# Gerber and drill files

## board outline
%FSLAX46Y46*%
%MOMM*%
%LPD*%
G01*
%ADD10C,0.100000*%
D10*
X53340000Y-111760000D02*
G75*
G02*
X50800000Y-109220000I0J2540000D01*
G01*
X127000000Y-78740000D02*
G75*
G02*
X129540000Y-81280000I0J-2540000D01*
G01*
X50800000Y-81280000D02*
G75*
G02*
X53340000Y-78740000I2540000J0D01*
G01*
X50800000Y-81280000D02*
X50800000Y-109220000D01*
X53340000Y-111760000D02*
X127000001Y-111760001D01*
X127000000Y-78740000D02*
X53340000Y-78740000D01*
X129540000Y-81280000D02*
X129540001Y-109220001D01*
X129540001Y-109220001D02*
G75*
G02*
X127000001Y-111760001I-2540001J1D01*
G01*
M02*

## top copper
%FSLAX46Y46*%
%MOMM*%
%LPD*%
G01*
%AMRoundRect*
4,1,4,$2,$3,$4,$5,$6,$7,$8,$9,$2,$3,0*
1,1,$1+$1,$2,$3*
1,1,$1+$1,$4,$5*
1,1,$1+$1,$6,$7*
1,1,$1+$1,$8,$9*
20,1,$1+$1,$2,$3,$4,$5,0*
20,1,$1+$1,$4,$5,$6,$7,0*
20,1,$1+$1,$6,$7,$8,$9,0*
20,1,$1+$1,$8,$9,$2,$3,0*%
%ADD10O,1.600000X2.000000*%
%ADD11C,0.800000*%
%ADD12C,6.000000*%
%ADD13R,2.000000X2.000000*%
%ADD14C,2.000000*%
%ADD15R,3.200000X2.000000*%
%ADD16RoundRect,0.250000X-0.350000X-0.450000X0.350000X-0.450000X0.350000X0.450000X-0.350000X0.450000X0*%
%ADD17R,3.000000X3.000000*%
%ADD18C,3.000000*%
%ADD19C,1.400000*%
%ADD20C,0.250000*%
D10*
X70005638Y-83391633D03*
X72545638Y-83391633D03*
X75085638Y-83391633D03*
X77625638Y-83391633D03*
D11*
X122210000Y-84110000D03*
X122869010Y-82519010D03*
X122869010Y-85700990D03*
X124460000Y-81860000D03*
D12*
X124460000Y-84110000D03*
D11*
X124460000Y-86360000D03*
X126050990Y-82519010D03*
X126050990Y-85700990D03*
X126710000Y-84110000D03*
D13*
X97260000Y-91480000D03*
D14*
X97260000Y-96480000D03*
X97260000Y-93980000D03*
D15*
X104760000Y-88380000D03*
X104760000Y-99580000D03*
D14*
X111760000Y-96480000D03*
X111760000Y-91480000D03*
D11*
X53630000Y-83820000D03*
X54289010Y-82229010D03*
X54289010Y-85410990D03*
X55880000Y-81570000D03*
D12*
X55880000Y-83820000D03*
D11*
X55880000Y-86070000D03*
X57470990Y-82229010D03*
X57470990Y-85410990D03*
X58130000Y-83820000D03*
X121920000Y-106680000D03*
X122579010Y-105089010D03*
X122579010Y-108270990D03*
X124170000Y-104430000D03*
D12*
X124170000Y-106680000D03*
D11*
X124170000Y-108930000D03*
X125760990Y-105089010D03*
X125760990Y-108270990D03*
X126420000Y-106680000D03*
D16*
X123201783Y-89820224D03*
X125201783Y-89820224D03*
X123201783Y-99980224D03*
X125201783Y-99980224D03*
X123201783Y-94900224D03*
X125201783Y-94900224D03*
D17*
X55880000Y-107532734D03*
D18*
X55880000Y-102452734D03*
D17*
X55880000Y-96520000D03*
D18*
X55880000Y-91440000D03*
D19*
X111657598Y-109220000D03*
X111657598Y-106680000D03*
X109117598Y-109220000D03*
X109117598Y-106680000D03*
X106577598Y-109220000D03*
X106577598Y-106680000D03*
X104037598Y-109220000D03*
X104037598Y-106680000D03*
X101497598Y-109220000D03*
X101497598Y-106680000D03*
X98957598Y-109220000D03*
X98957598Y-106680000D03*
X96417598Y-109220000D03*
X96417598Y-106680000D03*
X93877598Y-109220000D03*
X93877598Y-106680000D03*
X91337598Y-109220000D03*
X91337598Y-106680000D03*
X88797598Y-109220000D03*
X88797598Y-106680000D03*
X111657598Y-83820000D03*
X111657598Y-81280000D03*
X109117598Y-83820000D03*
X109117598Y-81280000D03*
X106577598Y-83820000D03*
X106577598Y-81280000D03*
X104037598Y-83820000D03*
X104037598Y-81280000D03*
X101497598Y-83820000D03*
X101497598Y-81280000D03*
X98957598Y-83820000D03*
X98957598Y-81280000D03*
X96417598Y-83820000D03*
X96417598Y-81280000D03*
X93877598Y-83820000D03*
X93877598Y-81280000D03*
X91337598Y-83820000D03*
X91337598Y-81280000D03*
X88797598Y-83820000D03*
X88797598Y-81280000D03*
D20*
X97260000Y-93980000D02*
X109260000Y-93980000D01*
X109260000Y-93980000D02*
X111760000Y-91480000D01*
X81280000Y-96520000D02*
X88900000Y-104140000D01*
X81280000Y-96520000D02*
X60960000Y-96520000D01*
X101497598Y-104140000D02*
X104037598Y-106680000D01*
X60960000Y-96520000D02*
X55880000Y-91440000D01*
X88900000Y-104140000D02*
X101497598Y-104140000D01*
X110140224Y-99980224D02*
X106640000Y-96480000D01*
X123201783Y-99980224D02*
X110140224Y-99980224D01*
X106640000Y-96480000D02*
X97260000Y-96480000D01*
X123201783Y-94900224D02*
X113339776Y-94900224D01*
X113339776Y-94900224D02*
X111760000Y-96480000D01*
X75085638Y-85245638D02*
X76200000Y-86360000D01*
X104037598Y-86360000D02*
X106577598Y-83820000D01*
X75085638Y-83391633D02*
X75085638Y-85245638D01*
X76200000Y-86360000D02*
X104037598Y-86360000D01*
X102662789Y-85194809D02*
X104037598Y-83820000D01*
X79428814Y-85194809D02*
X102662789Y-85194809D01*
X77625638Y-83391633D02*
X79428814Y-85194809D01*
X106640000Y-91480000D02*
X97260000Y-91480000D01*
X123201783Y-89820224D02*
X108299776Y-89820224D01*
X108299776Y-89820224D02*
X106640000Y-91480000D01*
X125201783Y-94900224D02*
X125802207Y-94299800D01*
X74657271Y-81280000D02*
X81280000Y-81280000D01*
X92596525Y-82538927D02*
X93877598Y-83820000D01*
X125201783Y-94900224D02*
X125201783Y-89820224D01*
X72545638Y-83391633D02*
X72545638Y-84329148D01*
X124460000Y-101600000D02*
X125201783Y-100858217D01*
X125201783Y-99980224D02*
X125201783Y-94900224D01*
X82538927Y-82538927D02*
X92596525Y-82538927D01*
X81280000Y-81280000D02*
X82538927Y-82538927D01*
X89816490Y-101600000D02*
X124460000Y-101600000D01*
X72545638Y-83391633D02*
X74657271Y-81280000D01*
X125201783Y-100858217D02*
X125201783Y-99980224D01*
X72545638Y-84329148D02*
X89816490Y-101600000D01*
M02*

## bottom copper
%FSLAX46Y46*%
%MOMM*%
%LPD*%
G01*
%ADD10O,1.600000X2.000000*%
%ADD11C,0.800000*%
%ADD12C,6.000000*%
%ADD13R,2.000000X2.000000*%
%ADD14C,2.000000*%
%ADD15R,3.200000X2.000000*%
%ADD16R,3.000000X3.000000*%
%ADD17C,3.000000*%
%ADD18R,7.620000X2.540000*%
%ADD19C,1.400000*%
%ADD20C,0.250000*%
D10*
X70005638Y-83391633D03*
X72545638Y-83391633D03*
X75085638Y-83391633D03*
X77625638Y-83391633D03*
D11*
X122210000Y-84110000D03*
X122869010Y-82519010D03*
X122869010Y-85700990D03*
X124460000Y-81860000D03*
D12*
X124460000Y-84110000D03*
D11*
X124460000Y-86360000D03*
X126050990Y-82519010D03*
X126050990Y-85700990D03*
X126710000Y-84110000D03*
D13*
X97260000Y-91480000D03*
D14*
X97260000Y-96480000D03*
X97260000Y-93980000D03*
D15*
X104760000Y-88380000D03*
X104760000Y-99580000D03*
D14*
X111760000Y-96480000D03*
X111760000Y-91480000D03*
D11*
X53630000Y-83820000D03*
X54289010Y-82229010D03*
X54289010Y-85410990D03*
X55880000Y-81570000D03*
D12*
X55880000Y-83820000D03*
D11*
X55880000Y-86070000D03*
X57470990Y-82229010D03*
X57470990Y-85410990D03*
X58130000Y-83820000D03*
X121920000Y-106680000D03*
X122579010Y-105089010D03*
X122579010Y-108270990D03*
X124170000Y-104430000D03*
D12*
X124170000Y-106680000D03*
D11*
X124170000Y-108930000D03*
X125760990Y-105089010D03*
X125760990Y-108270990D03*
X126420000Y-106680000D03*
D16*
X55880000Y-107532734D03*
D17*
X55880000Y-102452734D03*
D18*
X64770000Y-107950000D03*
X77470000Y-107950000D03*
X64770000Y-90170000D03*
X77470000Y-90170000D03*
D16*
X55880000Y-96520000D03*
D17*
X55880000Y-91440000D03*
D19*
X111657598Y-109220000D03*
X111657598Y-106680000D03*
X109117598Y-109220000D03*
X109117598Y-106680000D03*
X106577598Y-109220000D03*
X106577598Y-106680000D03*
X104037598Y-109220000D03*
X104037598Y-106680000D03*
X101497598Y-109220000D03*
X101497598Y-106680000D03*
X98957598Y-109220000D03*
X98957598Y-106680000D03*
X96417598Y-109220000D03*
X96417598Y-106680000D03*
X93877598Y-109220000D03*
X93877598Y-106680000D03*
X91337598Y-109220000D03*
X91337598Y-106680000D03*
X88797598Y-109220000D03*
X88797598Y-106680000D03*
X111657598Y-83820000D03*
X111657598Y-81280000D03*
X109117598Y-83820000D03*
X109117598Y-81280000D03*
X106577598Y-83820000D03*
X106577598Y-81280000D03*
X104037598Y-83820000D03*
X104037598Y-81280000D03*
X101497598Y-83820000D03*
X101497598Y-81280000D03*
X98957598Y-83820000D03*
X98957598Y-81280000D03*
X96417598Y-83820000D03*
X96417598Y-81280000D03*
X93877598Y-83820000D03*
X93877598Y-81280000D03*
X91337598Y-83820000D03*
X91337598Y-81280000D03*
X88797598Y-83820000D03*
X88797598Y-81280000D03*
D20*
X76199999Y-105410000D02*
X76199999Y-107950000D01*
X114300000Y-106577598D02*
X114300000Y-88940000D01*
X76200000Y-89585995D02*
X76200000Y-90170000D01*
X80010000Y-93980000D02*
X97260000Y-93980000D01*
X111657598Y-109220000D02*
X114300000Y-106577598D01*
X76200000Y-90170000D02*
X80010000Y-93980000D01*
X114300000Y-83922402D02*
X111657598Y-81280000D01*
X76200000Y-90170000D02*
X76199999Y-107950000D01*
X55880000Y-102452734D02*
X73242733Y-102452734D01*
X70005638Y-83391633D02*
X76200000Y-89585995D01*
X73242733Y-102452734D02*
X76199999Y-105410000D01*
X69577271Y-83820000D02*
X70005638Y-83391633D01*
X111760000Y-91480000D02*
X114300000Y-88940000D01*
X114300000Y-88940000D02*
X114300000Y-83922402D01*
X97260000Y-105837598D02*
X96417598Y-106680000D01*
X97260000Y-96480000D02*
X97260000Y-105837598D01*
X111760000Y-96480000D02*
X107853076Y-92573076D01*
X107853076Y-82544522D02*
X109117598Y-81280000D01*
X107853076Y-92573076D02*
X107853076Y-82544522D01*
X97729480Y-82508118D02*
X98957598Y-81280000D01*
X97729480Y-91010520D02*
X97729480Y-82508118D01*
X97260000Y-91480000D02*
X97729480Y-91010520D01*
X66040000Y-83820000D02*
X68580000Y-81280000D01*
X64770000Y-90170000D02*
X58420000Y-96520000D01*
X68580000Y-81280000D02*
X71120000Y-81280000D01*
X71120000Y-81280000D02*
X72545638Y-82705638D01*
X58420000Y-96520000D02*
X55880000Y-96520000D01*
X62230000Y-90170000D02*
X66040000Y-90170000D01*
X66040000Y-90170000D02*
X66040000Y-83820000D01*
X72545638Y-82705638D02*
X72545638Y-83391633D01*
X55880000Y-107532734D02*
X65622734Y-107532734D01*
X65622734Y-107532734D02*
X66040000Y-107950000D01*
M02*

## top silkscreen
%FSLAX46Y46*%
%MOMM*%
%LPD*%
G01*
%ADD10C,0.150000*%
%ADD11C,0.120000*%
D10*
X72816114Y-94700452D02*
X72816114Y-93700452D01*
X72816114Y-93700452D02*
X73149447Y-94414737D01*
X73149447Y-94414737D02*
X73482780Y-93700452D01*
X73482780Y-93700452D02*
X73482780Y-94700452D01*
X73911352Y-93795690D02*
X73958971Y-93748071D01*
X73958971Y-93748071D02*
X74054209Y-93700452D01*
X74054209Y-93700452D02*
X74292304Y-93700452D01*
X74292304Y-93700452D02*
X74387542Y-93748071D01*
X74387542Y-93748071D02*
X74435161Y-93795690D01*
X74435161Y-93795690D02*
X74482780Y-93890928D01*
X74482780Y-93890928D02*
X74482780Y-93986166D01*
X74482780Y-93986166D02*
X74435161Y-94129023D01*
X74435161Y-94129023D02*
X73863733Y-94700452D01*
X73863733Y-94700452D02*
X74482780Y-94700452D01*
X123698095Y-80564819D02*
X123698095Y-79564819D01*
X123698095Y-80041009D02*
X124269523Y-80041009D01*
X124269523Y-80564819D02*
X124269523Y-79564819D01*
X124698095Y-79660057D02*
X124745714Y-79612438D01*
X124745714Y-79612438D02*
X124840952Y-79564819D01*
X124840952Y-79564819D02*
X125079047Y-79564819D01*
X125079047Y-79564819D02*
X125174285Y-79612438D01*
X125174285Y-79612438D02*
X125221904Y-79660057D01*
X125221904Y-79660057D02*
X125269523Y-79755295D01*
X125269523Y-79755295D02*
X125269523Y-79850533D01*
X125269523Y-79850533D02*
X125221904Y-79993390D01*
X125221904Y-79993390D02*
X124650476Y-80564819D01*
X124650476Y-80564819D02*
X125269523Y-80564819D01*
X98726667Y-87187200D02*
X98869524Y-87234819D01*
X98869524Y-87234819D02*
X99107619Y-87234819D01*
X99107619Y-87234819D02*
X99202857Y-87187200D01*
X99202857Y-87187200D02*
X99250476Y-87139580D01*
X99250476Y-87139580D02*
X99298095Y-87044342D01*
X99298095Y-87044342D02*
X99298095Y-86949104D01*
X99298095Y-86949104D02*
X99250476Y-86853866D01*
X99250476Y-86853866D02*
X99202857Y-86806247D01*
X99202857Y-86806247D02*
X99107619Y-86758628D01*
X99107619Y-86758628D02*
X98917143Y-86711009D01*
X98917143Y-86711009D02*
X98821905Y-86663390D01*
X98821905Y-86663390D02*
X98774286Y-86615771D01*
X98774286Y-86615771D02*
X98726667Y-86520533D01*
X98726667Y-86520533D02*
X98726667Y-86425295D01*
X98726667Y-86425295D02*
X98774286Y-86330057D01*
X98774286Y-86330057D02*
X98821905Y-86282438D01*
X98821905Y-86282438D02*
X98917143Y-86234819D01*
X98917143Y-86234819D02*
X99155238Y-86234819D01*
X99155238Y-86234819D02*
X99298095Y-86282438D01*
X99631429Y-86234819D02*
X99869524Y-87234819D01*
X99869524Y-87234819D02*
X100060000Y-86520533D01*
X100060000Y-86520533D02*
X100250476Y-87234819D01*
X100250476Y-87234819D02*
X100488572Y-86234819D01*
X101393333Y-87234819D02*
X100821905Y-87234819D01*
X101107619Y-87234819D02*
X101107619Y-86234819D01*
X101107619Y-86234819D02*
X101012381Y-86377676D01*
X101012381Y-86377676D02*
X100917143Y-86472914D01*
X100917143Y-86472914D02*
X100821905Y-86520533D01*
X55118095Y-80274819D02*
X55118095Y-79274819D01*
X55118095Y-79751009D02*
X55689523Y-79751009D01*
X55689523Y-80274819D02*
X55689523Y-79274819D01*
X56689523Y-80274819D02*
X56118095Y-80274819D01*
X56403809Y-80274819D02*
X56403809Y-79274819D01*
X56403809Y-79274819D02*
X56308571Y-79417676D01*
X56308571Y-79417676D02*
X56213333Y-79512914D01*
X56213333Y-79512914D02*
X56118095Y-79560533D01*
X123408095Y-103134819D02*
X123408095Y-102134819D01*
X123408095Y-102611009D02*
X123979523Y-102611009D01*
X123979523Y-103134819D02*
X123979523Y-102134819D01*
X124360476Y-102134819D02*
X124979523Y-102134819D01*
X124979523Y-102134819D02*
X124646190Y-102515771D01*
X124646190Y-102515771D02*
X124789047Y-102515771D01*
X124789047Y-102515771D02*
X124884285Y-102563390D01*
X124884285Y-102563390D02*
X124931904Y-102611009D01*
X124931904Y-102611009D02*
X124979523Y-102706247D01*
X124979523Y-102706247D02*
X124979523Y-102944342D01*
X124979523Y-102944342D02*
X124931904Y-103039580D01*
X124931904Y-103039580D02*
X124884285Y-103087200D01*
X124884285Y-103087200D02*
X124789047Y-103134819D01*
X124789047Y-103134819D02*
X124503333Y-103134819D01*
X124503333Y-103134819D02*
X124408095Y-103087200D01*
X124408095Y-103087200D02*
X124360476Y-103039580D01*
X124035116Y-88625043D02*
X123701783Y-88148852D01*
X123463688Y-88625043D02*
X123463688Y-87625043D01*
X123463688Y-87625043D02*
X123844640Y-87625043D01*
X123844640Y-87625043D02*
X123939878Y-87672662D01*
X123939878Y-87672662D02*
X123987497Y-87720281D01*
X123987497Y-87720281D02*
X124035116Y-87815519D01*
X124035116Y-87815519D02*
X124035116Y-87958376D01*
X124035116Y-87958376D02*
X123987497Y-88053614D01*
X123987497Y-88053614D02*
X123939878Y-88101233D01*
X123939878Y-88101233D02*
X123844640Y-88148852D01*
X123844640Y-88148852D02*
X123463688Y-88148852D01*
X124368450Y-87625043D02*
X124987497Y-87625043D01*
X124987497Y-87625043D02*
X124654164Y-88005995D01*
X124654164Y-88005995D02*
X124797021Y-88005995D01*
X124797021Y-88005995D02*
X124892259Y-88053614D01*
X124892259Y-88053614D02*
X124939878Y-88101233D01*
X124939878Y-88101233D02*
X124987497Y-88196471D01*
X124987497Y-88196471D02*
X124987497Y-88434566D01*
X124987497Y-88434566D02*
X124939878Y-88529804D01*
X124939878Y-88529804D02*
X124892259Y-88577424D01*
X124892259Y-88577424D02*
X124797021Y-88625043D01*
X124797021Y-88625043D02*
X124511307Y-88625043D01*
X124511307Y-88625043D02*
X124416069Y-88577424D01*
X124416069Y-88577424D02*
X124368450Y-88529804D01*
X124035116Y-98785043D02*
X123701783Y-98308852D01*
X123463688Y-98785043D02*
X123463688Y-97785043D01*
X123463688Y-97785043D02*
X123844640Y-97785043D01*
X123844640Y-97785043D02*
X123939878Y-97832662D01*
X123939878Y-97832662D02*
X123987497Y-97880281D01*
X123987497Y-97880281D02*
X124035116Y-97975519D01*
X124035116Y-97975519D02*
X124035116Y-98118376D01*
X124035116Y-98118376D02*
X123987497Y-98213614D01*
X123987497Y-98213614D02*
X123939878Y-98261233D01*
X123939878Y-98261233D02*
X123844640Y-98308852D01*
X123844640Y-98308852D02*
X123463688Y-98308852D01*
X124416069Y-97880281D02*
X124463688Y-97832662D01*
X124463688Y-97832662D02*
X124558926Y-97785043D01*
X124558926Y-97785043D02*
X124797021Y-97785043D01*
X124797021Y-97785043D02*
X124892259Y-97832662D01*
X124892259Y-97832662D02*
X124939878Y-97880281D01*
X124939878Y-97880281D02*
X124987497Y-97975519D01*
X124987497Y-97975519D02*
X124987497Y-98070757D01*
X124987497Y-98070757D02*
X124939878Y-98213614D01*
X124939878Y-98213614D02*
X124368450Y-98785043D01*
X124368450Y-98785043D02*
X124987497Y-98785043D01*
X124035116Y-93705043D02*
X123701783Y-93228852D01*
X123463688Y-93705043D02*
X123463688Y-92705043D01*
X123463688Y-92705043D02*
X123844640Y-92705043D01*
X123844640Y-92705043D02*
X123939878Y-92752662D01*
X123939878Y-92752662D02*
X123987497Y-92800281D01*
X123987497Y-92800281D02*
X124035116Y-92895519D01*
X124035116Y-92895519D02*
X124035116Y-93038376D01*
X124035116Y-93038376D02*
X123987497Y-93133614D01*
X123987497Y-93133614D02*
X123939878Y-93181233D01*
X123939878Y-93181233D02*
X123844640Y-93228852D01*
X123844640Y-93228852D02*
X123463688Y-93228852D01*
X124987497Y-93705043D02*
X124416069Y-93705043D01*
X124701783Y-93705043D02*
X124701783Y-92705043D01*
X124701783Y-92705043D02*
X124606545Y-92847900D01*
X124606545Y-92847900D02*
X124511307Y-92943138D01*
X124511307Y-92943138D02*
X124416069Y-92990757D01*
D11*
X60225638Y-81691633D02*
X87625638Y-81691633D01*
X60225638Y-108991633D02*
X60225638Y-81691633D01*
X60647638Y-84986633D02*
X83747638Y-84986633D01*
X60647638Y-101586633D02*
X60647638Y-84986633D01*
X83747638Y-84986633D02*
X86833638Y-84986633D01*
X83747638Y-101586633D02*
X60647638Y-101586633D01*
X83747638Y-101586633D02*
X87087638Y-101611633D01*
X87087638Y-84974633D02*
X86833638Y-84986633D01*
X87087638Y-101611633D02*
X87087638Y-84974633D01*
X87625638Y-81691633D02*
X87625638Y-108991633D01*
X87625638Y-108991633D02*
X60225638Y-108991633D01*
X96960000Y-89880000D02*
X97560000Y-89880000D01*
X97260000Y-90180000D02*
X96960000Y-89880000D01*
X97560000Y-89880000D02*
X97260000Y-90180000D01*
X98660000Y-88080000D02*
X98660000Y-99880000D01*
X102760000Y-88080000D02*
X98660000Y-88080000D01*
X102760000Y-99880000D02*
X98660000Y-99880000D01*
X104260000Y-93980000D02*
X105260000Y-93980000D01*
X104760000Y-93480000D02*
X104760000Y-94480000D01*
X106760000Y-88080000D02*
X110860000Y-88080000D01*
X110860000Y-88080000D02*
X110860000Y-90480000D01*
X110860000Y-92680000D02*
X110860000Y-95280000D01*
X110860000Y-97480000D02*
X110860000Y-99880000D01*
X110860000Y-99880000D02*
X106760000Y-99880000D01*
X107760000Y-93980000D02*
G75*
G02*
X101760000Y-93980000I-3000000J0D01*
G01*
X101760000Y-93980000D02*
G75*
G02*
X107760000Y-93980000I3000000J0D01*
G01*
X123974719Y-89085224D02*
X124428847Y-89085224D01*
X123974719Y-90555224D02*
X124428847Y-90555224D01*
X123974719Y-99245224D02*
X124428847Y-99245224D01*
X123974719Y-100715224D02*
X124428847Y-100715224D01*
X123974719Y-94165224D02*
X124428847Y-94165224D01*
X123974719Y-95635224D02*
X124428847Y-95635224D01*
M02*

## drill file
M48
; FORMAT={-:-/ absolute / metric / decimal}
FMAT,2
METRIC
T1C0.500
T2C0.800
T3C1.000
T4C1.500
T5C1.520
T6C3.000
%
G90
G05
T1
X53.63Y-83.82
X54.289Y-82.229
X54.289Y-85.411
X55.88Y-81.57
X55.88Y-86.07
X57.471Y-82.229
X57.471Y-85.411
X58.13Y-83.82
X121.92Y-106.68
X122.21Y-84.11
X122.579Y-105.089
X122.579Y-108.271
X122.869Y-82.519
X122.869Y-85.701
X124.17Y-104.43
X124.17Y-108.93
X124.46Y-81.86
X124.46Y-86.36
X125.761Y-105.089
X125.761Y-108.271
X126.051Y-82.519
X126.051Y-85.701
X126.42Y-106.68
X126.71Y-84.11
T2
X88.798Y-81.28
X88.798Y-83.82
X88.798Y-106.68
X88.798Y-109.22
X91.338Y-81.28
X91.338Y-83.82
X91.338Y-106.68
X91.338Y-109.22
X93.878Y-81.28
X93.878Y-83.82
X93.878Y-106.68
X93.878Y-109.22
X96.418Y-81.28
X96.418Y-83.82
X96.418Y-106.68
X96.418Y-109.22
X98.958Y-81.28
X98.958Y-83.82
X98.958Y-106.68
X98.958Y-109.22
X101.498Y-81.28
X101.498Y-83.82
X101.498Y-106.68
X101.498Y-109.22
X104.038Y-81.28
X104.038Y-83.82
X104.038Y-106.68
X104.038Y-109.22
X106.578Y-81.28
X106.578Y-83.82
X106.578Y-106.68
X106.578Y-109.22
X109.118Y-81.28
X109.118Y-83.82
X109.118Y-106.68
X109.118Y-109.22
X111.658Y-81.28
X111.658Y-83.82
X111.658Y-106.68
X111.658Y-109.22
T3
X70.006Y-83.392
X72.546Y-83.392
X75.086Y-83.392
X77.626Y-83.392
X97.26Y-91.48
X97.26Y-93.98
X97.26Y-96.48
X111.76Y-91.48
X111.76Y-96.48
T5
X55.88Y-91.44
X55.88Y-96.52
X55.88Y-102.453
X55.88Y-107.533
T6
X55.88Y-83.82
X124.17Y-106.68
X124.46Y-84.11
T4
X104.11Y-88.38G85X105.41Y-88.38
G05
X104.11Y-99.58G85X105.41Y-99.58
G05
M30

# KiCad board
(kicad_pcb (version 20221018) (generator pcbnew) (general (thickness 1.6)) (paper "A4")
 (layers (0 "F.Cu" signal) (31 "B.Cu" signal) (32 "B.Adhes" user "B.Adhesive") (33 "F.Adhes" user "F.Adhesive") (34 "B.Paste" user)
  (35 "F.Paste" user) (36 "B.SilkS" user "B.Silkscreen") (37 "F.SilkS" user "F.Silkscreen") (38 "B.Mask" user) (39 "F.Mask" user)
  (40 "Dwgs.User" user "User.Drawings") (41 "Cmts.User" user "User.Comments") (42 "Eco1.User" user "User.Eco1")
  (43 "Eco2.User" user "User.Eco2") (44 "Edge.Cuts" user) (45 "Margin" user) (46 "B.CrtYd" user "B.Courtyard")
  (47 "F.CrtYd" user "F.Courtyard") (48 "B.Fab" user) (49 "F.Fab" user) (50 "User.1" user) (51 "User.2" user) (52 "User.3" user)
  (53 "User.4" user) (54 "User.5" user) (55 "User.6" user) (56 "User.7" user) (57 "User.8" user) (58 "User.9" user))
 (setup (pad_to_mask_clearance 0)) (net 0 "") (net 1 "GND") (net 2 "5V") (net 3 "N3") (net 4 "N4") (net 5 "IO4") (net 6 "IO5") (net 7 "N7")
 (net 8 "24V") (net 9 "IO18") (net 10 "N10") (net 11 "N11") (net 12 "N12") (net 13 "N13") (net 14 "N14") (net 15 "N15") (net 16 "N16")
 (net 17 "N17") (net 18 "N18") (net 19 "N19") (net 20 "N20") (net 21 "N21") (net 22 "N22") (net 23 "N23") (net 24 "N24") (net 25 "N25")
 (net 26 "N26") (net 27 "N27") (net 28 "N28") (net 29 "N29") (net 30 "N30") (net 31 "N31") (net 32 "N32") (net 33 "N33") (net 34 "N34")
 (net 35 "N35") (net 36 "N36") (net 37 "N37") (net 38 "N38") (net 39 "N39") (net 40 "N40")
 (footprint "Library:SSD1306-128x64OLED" (layer "F.Cu") (at 73.625638 93.991633)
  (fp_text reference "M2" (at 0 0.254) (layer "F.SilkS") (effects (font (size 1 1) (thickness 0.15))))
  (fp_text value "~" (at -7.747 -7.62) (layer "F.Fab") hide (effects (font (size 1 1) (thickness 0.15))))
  (fp_line (start -13.4 -12.3) (end 14 -12.3) (stroke (width 0.12) (type solid)) (layer "F.SilkS"))
  (fp_line (start -13.4 15) (end -13.4 -12.3) (stroke (width 0.12) (type solid)) (layer "F.SilkS"))
  (fp_line (start -12.978 -9.005) (end 10.122 -9.005) (stroke (width 0.12) (type solid)) (layer "F.SilkS"))
  (fp_line (start -12.978 7.595) (end -12.978 -9.005) (stroke (width 0.12) (type solid)) (layer "F.SilkS"))
  (fp_line (start 10.122 -9.005) (end 13.208 -9.005) (stroke (width 0.12) (type solid)) (layer "F.SilkS"))
  (fp_line (start 10.122 7.595) (end -12.978 7.595) (stroke (width 0.12) (type solid)) (layer "F.SilkS"))
  (fp_line (start 10.122 7.595) (end 13.462 7.62) (stroke (width 0.12) (type solid)) (layer "F.SilkS"))
  (fp_line (start 13.462 -9.017) (end 13.208 -9.005) (stroke (width 0.12) (type solid)) (layer "F.SilkS"))
  (fp_line (start 13.462 7.62) (end 13.462 -9.017) (stroke (width 0.12) (type solid)) (layer "F.SilkS"))
  (fp_line (start 14 -12.3) (end 14 15) (stroke (width 0.12) (type solid)) (layer "F.SilkS"))
  (fp_line (start 14 15) (end -13.4 15) (stroke (width 0.12) (type solid)) (layer "F.SilkS"))
  (pad "1" thru_hole oval (at -3.62 -10.6 90) (size 2 1.6) (drill 1) (layers "*.Cu" "*.Mask") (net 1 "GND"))
  (pad "2" thru_hole oval (at -1.08 -10.6 90) (size 2 1.6) (drill 1) (layers "*.Cu" "*.Mask") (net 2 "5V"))
  (pad "3" thru_hole oval (at 1.46 -10.6 90) (size 2 1.6) (drill 1) (layers "*.Cu" "*.Mask") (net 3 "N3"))
  (pad "4" thru_hole oval (at 4 -10.6 90) (size 2 1.6) (drill 1) (layers "*.Cu" "*.Mask") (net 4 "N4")))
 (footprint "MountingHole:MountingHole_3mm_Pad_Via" (layer "F.Cu") (at 124.46 84.11)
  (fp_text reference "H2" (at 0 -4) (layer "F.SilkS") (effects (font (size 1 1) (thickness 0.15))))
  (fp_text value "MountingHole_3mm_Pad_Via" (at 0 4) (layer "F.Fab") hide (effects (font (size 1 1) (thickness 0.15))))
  (pad "1" thru_hole circle (at -2.25 0) (size 0.8 0.8) (drill 0.5) (layers "*.Cu" "*.Mask"))
  (pad "1" thru_hole circle (at -1.59099 -1.59099) (size 0.8 0.8) (drill 0.5) (layers "*.Cu" "*.Mask"))
  (pad "1" thru_hole circle (at -1.59099 1.59099) (size 0.8 0.8) (drill 0.5) (layers "*.Cu" "*.Mask"))
  (pad "1" thru_hole circle (at 0 -2.25) (size 0.8 0.8) (drill 0.5) (layers "*.Cu" "*.Mask"))
  (pad "1" thru_hole circle (at 0 0) (size 6 6) (drill 3) (layers "*.Cu" "*.Mask"))
  (pad "1" thru_hole circle (at 0 2.25) (size 0.8 0.8) (drill 0.5) (layers "*.Cu" "*.Mask"))
  (pad "1" thru_hole circle (at 1.59099 -1.59099) (size 0.8 0.8) (drill 0.5) (layers "*.Cu" "*.Mask"))
  (pad "1" thru_hole circle (at 1.59099 1.59099) (size 0.8 0.8) (drill 0.5) (layers "*.Cu" "*.Mask"))
  (pad "1" thru_hole circle (at 2.25 0) (size 0.8 0.8) (drill 0.5) (layers "*.Cu" "*.Mask")))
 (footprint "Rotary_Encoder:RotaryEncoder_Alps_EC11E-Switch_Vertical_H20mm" (layer "F.Cu") (at 97.26 91.48)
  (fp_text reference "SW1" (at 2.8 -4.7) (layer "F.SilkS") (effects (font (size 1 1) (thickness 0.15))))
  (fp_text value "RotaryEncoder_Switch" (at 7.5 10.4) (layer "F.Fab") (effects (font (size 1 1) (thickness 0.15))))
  (fp_line (start -0.3 -1.6) (end 0.3 -1.6) (stroke (width 0.12) (type solid)) (layer "F.SilkS"))
  (fp_line (start 0 -1.3) (end -0.3 -1.6) (stroke (width 0.12) (type solid)) (layer "F.SilkS"))
  (fp_line (start 0.3 -1.6) (end 0 -1.3) (stroke (width 0.12) (type solid)) (layer "F.SilkS"))
  (fp_line (start 1.4 -3.4) (end 1.4 8.4) (stroke (width 0.12) (type solid)) (layer "F.SilkS"))
  (fp_line (start 5.5 -3.4) (end 1.4 -3.4) (stroke (width 0.12) (type solid)) (layer "F.SilkS"))
  (fp_line (start 5.5 8.4) (end 1.4 8.4) (stroke (width 0.12) (type solid)) (layer "F.SilkS"))
  (fp_line (start 7 2.5) (end 8 2.5) (stroke (width 0.12) (type solid)) (layer "F.SilkS"))
  (fp_line (start 7.5 2) (end 7.5 3) (stroke (width 0.12) (type solid)) (layer "F.SilkS"))
  (fp_line (start 9.5 -3.4) (end 13.6 -3.4) (stroke (width 0.12) (type solid)) (layer "F.SilkS"))
  (fp_line (start 13.6 -3.4) (end 13.6 -1) (stroke (width 0.12) (type solid)) (layer "F.SilkS"))
  (fp_line (start 13.6 1.2) (end 13.6 3.8) (stroke (width 0.12) (type solid)) (layer "F.SilkS"))
  (fp_line (start 13.6 6) (end 13.6 8.4) (stroke (width 0.12) (type solid)) (layer "F.SilkS"))
  (fp_line (start 13.6 8.4) (end 9.5 8.4) (stroke (width 0.12) (type solid)) (layer "F.SilkS"))
  (fp_circle (center 7.5 2.5) (end 10.5 2.5) (stroke (width 0.12) (type solid)) (fill none) (layer "F.SilkS"))
  (pad "A" thru_hole rect (at 0 0) (size 2 2) (drill 1) (layers "*.Cu" "*.Mask") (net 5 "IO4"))
  (pad "B" thru_hole circle (at 0 5) (size 2 2) (drill 1) (layers "*.Cu" "*.Mask") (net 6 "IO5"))
  (pad "C" thru_hole circle (at 0 2.5) (size 2 2) (drill 1) (layers "*.Cu" "*.Mask") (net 1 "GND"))
  (pad "MP" thru_hole rect (at 7.5 -3.1) (size 3.2 2) (drill oval 2.8 1.5) (layers "*.Cu" "*.Mask"))
  (pad "MP" thru_hole rect (at 7.5 8.1) (size 3.2 2) (drill oval 2.8 1.5) (layers "*.Cu" "*.Mask"))
  (pad "S1" thru_hole circle (at 14.5 5) (size 2 2) (drill 1) (layers "*.Cu" "*.Mask") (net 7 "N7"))
  (pad "S2" thru_hole circle (at 14.5 0) (size 2 2) (drill 1) (layers "*.Cu" "*.Mask") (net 1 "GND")))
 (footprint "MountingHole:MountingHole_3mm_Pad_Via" (layer "F.Cu") (at 55.88 83.82)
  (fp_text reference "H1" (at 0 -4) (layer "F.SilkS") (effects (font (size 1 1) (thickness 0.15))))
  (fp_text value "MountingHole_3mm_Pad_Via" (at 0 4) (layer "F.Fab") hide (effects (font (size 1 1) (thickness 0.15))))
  (pad "1" thru_hole circle (at -2.25 0) (size 0.8 0.8) (drill 0.5) (layers "*.Cu" "*.Mask"))
  (pad "1" thru_hole circle (at -1.59099 -1.59099) (size 0.8 0.8) (drill 0.5) (layers "*.Cu" "*.Mask"))
  (pad "1" thru_hole circle (at -1.59099 1.59099) (size 0.8 0.8) (drill 0.5) (layers "*.Cu" "*.Mask"))
  (pad "1" thru_hole circle (at 0 -2.25) (size 0.8 0.8) (drill 0.5) (layers "*.Cu" "*.Mask"))
  (pad "1" thru_hole circle (at 0 0) (size 6 6) (drill 3) (layers "*.Cu" "*.Mask"))
  (pad "1" thru_hole circle (at 0 2.25) (size 0.8 0.8) (drill 0.5) (layers "*.Cu" "*.Mask"))
  (pad "1" thru_hole circle (at 1.59099 -1.59099) (size 0.8 0.8) (drill 0.5) (layers "*.Cu" "*.Mask"))
  (pad "1" thru_hole circle (at 1.59099 1.59099) (size 0.8 0.8) (drill 0.5) (layers "*.Cu" "*.Mask"))
  (pad "1" thru_hole circle (at 2.25 0) (size 0.8 0.8) (drill 0.5) (layers "*.Cu" "*.Mask")))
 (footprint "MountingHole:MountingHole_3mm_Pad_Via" (layer "F.Cu") (at 124.17 106.68)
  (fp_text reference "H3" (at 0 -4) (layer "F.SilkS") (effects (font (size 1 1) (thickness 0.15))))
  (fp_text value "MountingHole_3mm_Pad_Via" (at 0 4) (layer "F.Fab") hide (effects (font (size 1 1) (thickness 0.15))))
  (pad "1" thru_hole circle (at -2.25 0) (size 0.8 0.8) (drill 0.5) (layers "*.Cu" "*.Mask"))
  (pad "1" thru_hole circle (at -1.59099 -1.59099) (size 0.8 0.8) (drill 0.5) (layers "*.Cu" "*.Mask"))
  (pad "1" thru_hole circle (at -1.59099 1.59099) (size 0.8 0.8) (drill 0.5) (layers "*.Cu" "*.Mask"))
  (pad "1" thru_hole circle (at 0 -2.25) (size 0.8 0.8) (drill 0.5) (layers "*.Cu" "*.Mask"))
  (pad "1" thru_hole circle (at 0 0) (size 6 6) (drill 3) (layers "*.Cu" "*.Mask"))
  (pad "1" thru_hole circle (at 0 2.25) (size 0.8 0.8) (drill 0.5) (layers "*.Cu" "*.Mask"))
  (pad "1" thru_hole circle (at 1.59099 -1.59099) (size 0.8 0.8) (drill 0.5) (layers "*.Cu" "*.Mask"))
  (pad "1" thru_hole circle (at 1.59099 1.59099) (size 0.8 0.8) (drill 0.5) (layers "*.Cu" "*.Mask"))
  (pad "1" thru_hole circle (at 2.25 0) (size 0.8 0.8) (drill 0.5) (layers "*.Cu" "*.Mask")))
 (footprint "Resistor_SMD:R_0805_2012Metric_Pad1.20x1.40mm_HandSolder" (layer "F.Cu") (at 124.201783 89.820224)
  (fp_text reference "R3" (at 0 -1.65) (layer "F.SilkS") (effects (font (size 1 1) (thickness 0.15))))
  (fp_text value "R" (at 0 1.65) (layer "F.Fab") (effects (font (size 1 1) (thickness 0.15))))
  (fp_line (start -0.227064 -0.735) (end 0.227064 -0.735) (stroke (width 0.12) (type solid)) (layer "F.SilkS"))
  (fp_line (start -0.227064 0.735) (end 0.227064 0.735) (stroke (width 0.12) (type solid)) (layer "F.SilkS"))
  (pad "1" smd roundrect (at -1 0) (size 1.2 1.4) (layers "F.Cu" "F.Paste" "F.Mask") (roundrect_rratio 0.208333) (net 5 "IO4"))
  (pad "2" smd roundrect (at 1 0) (size 1.2 1.4) (layers "F.Cu" "F.Paste" "F.Mask") (roundrect_rratio 0.208333) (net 2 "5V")))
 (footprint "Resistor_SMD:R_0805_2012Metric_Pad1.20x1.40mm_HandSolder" (layer "F.Cu") (at 124.201783 99.980224)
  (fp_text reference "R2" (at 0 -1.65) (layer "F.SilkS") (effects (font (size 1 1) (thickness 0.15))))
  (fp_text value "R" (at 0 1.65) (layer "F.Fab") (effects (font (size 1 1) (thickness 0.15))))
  (fp_line (start -0.227064 -0.735) (end 0.227064 -0.735) (stroke (width 0.12) (type solid)) (layer "F.SilkS"))
  (fp_line (start -0.227064 0.735) (end 0.227064 0.735) (stroke (width 0.12) (type solid)) (layer "F.SilkS"))
  (pad "1" smd roundrect (at -1 0) (size 1.2 1.4) (layers "F.Cu" "F.Paste" "F.Mask") (roundrect_rratio 0.208333) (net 6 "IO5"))
  (pad "2" smd roundrect (at 1 0) (size 1.2 1.4) (layers "F.Cu" "F.Paste" "F.Mask") (roundrect_rratio 0.208333) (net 2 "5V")))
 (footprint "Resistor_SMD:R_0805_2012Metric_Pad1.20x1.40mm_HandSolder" (layer "F.Cu") (at 124.201783 94.900224)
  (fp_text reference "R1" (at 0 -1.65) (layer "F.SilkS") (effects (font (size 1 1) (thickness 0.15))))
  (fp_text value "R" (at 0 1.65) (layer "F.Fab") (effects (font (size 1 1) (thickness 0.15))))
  (fp_line (start -0.227064 -0.735) (end 0.227064 -0.735) (stroke (width 0.12) (type solid)) (layer "F.SilkS"))
  (fp_line (start -0.227064 0.735) (end 0.227064 0.735) (stroke (width 0.12) (type solid)) (layer "F.SilkS"))
  (pad "1" smd roundrect (at -1 0) (size 1.2 1.4) (layers "F.Cu" "F.Paste" "F.Mask") (roundrect_rratio 0.208333) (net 7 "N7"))
  (pad "2" smd roundrect (at 1 0) (size 1.2 1.4) (layers "F.Cu" "F.Paste" "F.Mask") (roundrect_rratio 0.208333) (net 2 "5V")))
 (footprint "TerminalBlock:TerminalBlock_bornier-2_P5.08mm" (layer "B.Cu") (at 55.88 107.532734 90)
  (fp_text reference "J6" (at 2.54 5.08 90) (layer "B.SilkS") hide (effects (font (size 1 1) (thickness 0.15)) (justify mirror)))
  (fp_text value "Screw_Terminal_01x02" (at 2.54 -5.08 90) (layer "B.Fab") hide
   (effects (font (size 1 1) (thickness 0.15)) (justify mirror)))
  (pad "1" thru_hole rect (at 0 0 90) (size 3 3) (drill 1.52) (layers "*.Cu" "*.Mask") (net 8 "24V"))
  (pad "2" thru_hole circle (at 5.08 0 90) (size 3 3) (drill 1.52) (layers "*.Cu" "*.Mask") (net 1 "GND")))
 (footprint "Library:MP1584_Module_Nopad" (layer "B.Cu") (at 71.12 99.06 -90)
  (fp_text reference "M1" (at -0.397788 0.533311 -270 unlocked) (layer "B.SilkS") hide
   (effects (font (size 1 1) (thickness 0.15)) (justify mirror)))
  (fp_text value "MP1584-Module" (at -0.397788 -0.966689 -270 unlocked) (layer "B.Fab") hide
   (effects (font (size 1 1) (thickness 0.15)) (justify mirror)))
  (pad "1" smd rect (at 8.89 6.35 90) (size 2.54 7.62) (layers "B.Cu" "B.Paste" "B.Mask") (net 8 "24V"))
  (pad "2" smd rect (at 8.89 -6.35 270) (size 2.54 7.62) (layers "B.Cu" "B.Paste" "B.Mask") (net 1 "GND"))
  (pad "3" smd rect (at -8.89 6.35 90) (size 2.54 7.62) (layers "B.Cu" "B.Paste" "B.Mask") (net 2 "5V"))
  (pad "4" smd rect (at -8.89 -6.35 270) (size 2.54 7.62) (layers "B.Cu" "B.Paste" "B.Mask") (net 1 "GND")))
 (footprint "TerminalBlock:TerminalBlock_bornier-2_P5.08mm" (layer "B.Cu") (at 55.88 96.52 90)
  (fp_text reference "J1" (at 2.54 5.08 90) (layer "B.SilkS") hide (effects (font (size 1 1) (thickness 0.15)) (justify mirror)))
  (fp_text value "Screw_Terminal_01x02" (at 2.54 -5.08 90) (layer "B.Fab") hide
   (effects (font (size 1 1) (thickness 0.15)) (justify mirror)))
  (pad "1" thru_hole rect (at 0 0 90) (size 3 3) (drill 1.52) (layers "*.Cu" "*.Mask") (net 2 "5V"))
  (pad "2" thru_hole circle (at 5.08 0 90) (size 3 3) (drill 1.52) (layers "*.Cu" "*.Mask") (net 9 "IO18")))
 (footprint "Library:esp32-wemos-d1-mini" (layer "B.Cu") (at 100.227598 95.25 90)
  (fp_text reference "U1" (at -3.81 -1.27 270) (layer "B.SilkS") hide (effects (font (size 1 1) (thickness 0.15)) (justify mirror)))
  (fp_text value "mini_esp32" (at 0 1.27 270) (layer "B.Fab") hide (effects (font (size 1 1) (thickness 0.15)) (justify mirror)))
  (pad "1" thru_hole circle (at -13.97 11.43 180) (size 1.4 1.4) (drill 0.8) (layers "*.Cu" "*.Mask") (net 1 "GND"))
  (pad "2" thru_hole circle (at -11.43 11.43 180) (size 1.4 1.4) (drill 0.8) (layers "*.Cu" "*.Mask") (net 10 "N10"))
  (pad "3" thru_hole circle (at -13.97 8.89 180) (size 1.4 1.4) (drill 0.8) (layers "*.Cu" "*.Mask") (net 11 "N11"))
  (pad "4" thru_hole circle (at -11.43 8.89 180) (size 1.4 1.4) (drill 0.8) (layers "*.Cu" "*.Mask") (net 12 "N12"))
  (pad "5" thru_hole circle (at -13.97 6.35 180) (size 1.4 1.4) (drill 0.8) (layers "*.Cu" "*.Mask") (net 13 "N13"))
  (pad "6" thru_hole circle (at -11.43 6.35 180) (size 1.4 1.4) (drill 0.8) (layers "*.Cu" "*.Mask") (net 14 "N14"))
  (pad "7" thru_hole circle (at -13.97 3.81 180) (size 1.4 1.4) (drill 0.8) (layers "*.Cu" "*.Mask") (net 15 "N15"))
  (pad "8" thru_hole circle (at -11.43 3.81 180) (size 1.4 1.4) (drill 0.8) (layers "*.Cu" "*.Mask") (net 9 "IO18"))
  (pad "9" thru_hole circle (at -13.97 1.27 180) (size 1.4 1.4) (drill 0.8) (layers "*.Cu" "*.Mask") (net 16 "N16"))
  (pad "10" thru_hole circle (at -11.43 1.27 180) (size 1.4 1.4) (drill 0.8) (layers "*.Cu" "*.Mask") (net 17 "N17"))
  (pad "11" thru_hole circle (at -13.97 -1.27 180) (size 1.4 1.4) (drill 0.8) (layers "*.Cu" "*.Mask") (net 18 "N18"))
  (pad "12" thru_hole circle (at -11.43 -1.27 180) (size 1.4 1.4) (drill 0.8) (layers "*.Cu" "*.Mask") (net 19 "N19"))
  (pad "13" thru_hole circle (at -13.97 -3.81 180) (size 1.4 1.4) (drill 0.8) (layers "*.Cu" "*.Mask") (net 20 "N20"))
  (pad "14" thru_hole circle (at -11.43 -3.81 180) (size 1.4 1.4) (drill 0.8) (layers "*.Cu" "*.Mask") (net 6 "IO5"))
  (pad "15" thru_hole circle (at -13.97 -6.35 180) (size 1.4 1.4) (drill 0.8) (layers "*.Cu" "*.Mask") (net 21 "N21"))
  (pad "16" thru_hole circle (at -11.43 -6.35 180) (size 1.4 1.4) (drill 0.8) (layers "*.Cu" "*.Mask") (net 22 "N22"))
  (pad "17" thru_hole circle (at -13.97 -8.89 180) (size 1.4 1.4) (drill 0.8) (layers "*.Cu" "*.Mask") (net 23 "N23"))
  (pad "18" thru_hole circle (at -11.43 -8.89 180) (size 1.4 1.4) (drill 0.8) (layers "*.Cu" "*.Mask") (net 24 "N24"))
  (pad "19" thru_hole circle (at -13.97 -11.43 180) (size 1.4 1.4) (drill 0.8) (layers "*.Cu" "*.Mask") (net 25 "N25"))
  (pad "20" thru_hole circle (at -11.43 -11.43 180) (size 1.4 1.4) (drill 0.8) (layers "*.Cu" "*.Mask") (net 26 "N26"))
  (pad "21" thru_hole circle (at 11.43 11.43 180) (size 1.4 1.4) (drill 0.8) (layers "*.Cu" "*.Mask") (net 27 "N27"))
  (pad "22" thru_hole circle (at 13.97 11.43 180) (size 1.4 1.4) (drill 0.8) (layers "*.Cu" "*.Mask") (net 1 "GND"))
  (pad "23" thru_hole circle (at 11.43 8.89 180) (size 1.4 1.4) (drill 0.8) (layers "*.Cu" "*.Mask") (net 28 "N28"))
  (pad "24" thru_hole circle (at 13.97 8.89 180) (size 1.4 1.4) (drill 0.8) (layers "*.Cu" "*.Mask") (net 7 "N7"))
  (pad "25" thru_hole circle (at 11.43 6.35 180) (size 1.4 1.4) (drill 0.8) (layers "*.Cu" "*.Mask") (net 3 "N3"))
  (pad "26" thru_hole circle (at 13.97 6.35 180) (size 1.4 1.4) (drill 0.8) (layers "*.Cu" "*.Mask") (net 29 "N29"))
  (pad "27" thru_hole circle (at 11.43 3.81 180) (size 1.4 1.4) (drill 0.8) (layers "*.Cu" "*.Mask") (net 4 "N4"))
  (pad "28" thru_hole circle (at 13.97 3.81 180) (size 1.4 1.4) (drill 0.8) (layers "*.Cu" "*.Mask") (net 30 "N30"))
  (pad "29" thru_hole circle (at 11.43 1.27 180) (size 1.4 1.4) (drill 0.8) (layers "*.Cu" "*.Mask") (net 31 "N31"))
  (pad "30" thru_hole circle (at 13.97 1.27 180) (size 1.4 1.4) (drill 0.8) (layers "*.Cu" "*.Mask") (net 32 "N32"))
  (pad "31" thru_hole circle (at 11.43 -1.27 180) (size 1.4 1.4) (drill 0.8) (layers "*.Cu" "*.Mask") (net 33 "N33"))
  (pad "32" thru_hole circle (at 13.97 -1.27 180) (size 1.4 1.4) (drill 0.8) (layers "*.Cu" "*.Mask") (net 5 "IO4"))
  (pad "33" thru_hole circle (at 11.43 -3.81 180) (size 1.4 1.4) (drill 0.8) (layers "*.Cu" "*.Mask") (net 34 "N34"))
  (pad "34" thru_hole circle (at 13.97 -3.81 180) (size 1.4 1.4) (drill 0.8) (layers "*.Cu" "*.Mask") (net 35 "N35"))
  (pad "35" thru_hole circle (at 11.43 -6.35 180) (size 1.4 1.4) (drill 0.8) (layers "*.Cu" "*.Mask") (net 2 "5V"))
  (pad "36" thru_hole circle (at 13.97 -6.35 180) (size 1.4 1.4) (drill 0.8) (layers "*.Cu" "*.Mask") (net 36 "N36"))
  (pad "37" thru_hole circle (at 11.43 -8.89 180) (size 1.4 1.4) (drill 0.8) (layers "*.Cu" "*.Mask") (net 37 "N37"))
  (pad "38" thru_hole circle (at 13.97 -8.89 180) (size 1.4 1.4) (drill 0.8) (layers "*.Cu" "*.Mask") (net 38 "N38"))
  (pad "39" thru_hole circle (at 11.43 -11.43 180) (size 1.4 1.4) (drill 0.8) (layers "*.Cu" "*.Mask") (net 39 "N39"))
  (pad "40" thru_hole circle (at 13.97 -11.43 180) (size 1.4 1.4) (drill 0.8) (layers "*.Cu" "*.Mask") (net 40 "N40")))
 (gr_arc (start 53.34 111.76) (mid 51.543949 111.016051) (end 50.8 109.22) (stroke (width 0.1) (type default)) (layer "Edge.Cuts"))
 (gr_arc (start 127 78.74) (mid 128.796051 79.483949) (end 129.54 81.28) (stroke (width 0.1) (type default)) (layer "Edge.Cuts"))
 (gr_arc (start 50.8 81.28) (mid 51.543949 79.483949) (end 53.34 78.74) (stroke (width 0.1) (type default)) (layer "Edge.Cuts"))
 (gr_line (start 50.8 81.28) (end 50.8 109.22) (stroke (width 0.1) (type default)) (layer "Edge.Cuts"))
 (gr_line (start 53.34 111.76) (end 127.000001 111.760001) (stroke (width 0.1) (type default)) (layer "Edge.Cuts"))
 (gr_line (start 127 78.74) (end 53.34 78.74) (stroke (width 0.1) (type default)) (layer "Edge.Cuts"))
 (gr_line (start 129.54 81.28) (end 129.540001 109.220001) (stroke (width 0.1) (type default)) (layer "Edge.Cuts"))
 (gr_arc (start 129.540001 109.220001) (mid 128.796052 111.016052) (end 127.000001 111.760001) (stroke (width 0.1) (type default))
  (layer "Edge.Cuts"))
 (segment (start 97.26 93.98) (end 109.26 93.98) (width 0.25) (layer "F.Cu") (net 1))
 (segment (start 109.26 93.98) (end 111.76 91.48) (width 0.25) (layer "F.Cu") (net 1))
 (segment (start 76.199999 105.41) (end 76.199999 107.95) (width 0.25) (layer "B.Cu") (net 1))
 (segment (start 114.3 106.577598) (end 114.3 88.94) (width 0.25) (layer "B.Cu") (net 1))
 (segment (start 76.2 89.585995) (end 76.2 90.17) (width 0.25) (layer "B.Cu") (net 1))
 (segment (start 80.01 93.98) (end 97.26 93.98) (width 0.25) (layer "B.Cu") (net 1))
 (segment (start 111.657598 109.22) (end 114.3 106.577598) (width 0.25) (layer "B.Cu") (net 1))
 (segment (start 76.2 90.17) (end 80.01 93.98) (width 0.25) (layer "B.Cu") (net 1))
 (segment (start 114.3 83.922402) (end 111.657598 81.28) (width 0.25) (layer "B.Cu") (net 1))
 (segment (start 76.2 90.17) (end 76.199999 107.95) (width 0.25) (layer "B.Cu") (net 1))
 (segment (start 55.88 102.452734) (end 73.242733 102.452734) (width 0.25) (layer "B.Cu") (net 1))
 (segment (start 70.005638 83.391633) (end 76.2 89.585995) (width 0.25) (layer "B.Cu") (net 1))
 (segment (start 73.242733 102.452734) (end 76.199999 105.41) (width 0.25) (layer "B.Cu") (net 1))
 (segment (start 69.577271 83.82) (end 70.005638 83.391633) (width 0.25) (layer "B.Cu") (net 1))
 (segment (start 111.76 91.48) (end 114.3 88.94) (width 0.25) (layer "B.Cu") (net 1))
 (segment (start 114.3 88.94) (end 114.3 83.922402) (width 0.25) (layer "B.Cu") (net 1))
 (segment (start 81.28 96.52) (end 88.9 104.14) (width 0.25) (layer "F.Cu") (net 9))
 (segment (start 81.28 96.52) (end 60.96 96.52) (width 0.25) (layer "F.Cu") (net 9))
 (segment (start 101.497598 104.14) (end 104.037598 106.68) (width 0.25) (layer "F.Cu") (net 9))
 (segment (start 60.96 96.52) (end 55.88 91.44) (width 0.25) (layer "F.Cu") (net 9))
 (segment (start 88.9 104.14) (end 101.497598 104.14) (width 0.25) (layer "F.Cu") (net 9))
 (segment (start 110.140224 99.980224) (end 106.64 96.48) (width 0.25) (layer "F.Cu") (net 6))
 (segment (start 123.201783 99.980224) (end 110.140224 99.980224) (width 0.25) (layer "F.Cu") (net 6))
 (segment (start 106.64 96.48) (end 97.26 96.48) (width 0.25) (layer "F.Cu") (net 6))
 (segment (start 97.26 105.837598) (end 96.417598 106.68) (width 0.25) (layer "B.Cu") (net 6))
 (segment (start 97.26 96.48) (end 97.26 105.837598) (width 0.25) (layer "B.Cu") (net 6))
 (segment (start 123.201783 94.900224) (end 113.339776 94.900224) (width 0.25) (layer "F.Cu") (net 7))
 (segment (start 113.339776 94.900224) (end 111.76 96.48) (width 0.25) (layer "F.Cu") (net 7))
 (segment (start 111.76 96.48) (end 107.853076 92.573076) (width 0.25) (layer "B.Cu") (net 7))
 (segment (start 107.853076 82.544522) (end 109.117598 81.28) (width 0.25) (layer "B.Cu") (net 7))
 (segment (start 107.853076 92.573076) (end 107.853076 82.544522) (width 0.25) (layer "B.Cu") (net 7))
 (segment (start 75.085638 85.245638) (end 76.2 86.36) (width 0.25) (layer "F.Cu") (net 3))
 (segment (start 104.037598 86.36) (end 106.577598 83.82) (width 0.25) (layer "F.Cu") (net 3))
 (segment (start 75.085638 83.391633) (end 75.085638 85.245638) (width 0.25) (layer "F.Cu") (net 3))
 (segment (start 76.2 86.36) (end 104.037598 86.36) (width 0.25) (layer "F.Cu") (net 3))
 (segment (start 102.662789 85.194809) (end 104.037598 83.82) (width 0.25) (layer "F.Cu") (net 4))
 (segment (start 79.428814 85.194809) (end 102.662789 85.194809) (width 0.25) (layer "F.Cu") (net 4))
 (segment (start 77.625638 83.391633) (end 79.428814 85.194809) (width 0.25) (layer "F.Cu") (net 4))
 (segment (start 106.64 91.48) (end 97.26 91.48) (width 0.25) (layer "F.Cu") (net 5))
 (segment (start 123.201783 89.820224) (end 108.299776 89.820224) (width 0.25) (layer "F.Cu") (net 5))
 (segment (start 108.299776 89.820224) (end 106.64 91.48) (width 0.25) (layer "F.Cu") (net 5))
 (segment (start 97.72948 82.508118) (end 98.957598 81.28) (width 0.25) (layer "B.Cu") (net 5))
 (segment (start 97.72948 91.01052) (end 97.72948 82.508118) (width 0.25) (layer "B.Cu") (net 5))
 (segment (start 97.26 91.48) (end 97.72948 91.01052) (width 0.25) (layer "B.Cu") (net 5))
 (segment (start 125.201783 94.900224) (end 125.802207 94.2998) (width 0.25) (layer "F.Cu") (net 2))
 (segment (start 74.657271 81.28) (end 81.28 81.28) (width 0.25) (layer "F.Cu") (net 2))
 (segment (start 92.596525 82.538927) (end 93.877598 83.82) (width 0.25) (layer "F.Cu") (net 2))
 (segment (start 125.201783 94.900224) (end 125.201783 89.820224) (width 0.25) (layer "F.Cu") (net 2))
 (segment (start 72.545638 83.391633) (end 72.545638 84.329148) (width 0.25) (layer "F.Cu") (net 2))
 (segment (start 124.46 101.6) (end 125.201783 100.858217) (width 0.25) (layer "F.Cu") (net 2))
 (segment (start 125.201783 99.980224) (end 125.201783 94.900224) (width 0.25) (layer "F.Cu") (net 2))
 (segment (start 82.538927 82.538927) (end 92.596525 82.538927) (width 0.25) (layer "F.Cu") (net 2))
 (segment (start 81.28 81.28) (end 82.538927 82.538927) (width 0.25) (layer "F.Cu") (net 2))
 (segment (start 89.81649 101.6) (end 124.46 101.6) (width 0.25) (layer "F.Cu") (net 2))
 (segment (start 72.545638 83.391633) (end 74.657271 81.28) (width 0.25) (layer "F.Cu") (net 2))
 (segment (start 125.201783 100.858217) (end 125.201783 99.980224) (width 0.25) (layer "F.Cu") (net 2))
 (segment (start 72.545638 84.329148) (end 89.81649 101.6) (width 0.25) (layer "F.Cu") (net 2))
 (segment (start 66.04 83.82) (end 68.58 81.28) (width 0.25) (layer "B.Cu") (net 2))
 (segment (start 64.77 90.17) (end 58.42 96.52) (width 0.25) (layer "B.Cu") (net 2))
 (segment (start 68.58 81.28) (end 71.12 81.28) (width 0.25) (layer "B.Cu") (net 2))
 (segment (start 71.12 81.28) (end 72.545638 82.705638) (width 0.25) (layer "B.Cu") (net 2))
 (segment (start 58.42 96.52) (end 55.88 96.52) (width 0.25) (layer "B.Cu") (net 2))
 (segment (start 62.23 90.17) (end 66.04 90.17) (width 0.25) (layer "B.Cu") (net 2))
 (segment (start 66.04 90.17) (end 66.04 83.82) (width 0.25) (layer "B.Cu") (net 2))
 (segment (start 72.545638 82.705638) (end 72.545638 83.391633) (width 0.25) (layer "B.Cu") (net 2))
 (segment (start 55.88 107.532734) (end 65.622734 107.532734) (width 0.25) (layer "B.Cu") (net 8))
 (segment (start 65.622734 107.532734) (end 66.04 107.95) (width 0.25) (layer "B.Cu") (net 8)))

